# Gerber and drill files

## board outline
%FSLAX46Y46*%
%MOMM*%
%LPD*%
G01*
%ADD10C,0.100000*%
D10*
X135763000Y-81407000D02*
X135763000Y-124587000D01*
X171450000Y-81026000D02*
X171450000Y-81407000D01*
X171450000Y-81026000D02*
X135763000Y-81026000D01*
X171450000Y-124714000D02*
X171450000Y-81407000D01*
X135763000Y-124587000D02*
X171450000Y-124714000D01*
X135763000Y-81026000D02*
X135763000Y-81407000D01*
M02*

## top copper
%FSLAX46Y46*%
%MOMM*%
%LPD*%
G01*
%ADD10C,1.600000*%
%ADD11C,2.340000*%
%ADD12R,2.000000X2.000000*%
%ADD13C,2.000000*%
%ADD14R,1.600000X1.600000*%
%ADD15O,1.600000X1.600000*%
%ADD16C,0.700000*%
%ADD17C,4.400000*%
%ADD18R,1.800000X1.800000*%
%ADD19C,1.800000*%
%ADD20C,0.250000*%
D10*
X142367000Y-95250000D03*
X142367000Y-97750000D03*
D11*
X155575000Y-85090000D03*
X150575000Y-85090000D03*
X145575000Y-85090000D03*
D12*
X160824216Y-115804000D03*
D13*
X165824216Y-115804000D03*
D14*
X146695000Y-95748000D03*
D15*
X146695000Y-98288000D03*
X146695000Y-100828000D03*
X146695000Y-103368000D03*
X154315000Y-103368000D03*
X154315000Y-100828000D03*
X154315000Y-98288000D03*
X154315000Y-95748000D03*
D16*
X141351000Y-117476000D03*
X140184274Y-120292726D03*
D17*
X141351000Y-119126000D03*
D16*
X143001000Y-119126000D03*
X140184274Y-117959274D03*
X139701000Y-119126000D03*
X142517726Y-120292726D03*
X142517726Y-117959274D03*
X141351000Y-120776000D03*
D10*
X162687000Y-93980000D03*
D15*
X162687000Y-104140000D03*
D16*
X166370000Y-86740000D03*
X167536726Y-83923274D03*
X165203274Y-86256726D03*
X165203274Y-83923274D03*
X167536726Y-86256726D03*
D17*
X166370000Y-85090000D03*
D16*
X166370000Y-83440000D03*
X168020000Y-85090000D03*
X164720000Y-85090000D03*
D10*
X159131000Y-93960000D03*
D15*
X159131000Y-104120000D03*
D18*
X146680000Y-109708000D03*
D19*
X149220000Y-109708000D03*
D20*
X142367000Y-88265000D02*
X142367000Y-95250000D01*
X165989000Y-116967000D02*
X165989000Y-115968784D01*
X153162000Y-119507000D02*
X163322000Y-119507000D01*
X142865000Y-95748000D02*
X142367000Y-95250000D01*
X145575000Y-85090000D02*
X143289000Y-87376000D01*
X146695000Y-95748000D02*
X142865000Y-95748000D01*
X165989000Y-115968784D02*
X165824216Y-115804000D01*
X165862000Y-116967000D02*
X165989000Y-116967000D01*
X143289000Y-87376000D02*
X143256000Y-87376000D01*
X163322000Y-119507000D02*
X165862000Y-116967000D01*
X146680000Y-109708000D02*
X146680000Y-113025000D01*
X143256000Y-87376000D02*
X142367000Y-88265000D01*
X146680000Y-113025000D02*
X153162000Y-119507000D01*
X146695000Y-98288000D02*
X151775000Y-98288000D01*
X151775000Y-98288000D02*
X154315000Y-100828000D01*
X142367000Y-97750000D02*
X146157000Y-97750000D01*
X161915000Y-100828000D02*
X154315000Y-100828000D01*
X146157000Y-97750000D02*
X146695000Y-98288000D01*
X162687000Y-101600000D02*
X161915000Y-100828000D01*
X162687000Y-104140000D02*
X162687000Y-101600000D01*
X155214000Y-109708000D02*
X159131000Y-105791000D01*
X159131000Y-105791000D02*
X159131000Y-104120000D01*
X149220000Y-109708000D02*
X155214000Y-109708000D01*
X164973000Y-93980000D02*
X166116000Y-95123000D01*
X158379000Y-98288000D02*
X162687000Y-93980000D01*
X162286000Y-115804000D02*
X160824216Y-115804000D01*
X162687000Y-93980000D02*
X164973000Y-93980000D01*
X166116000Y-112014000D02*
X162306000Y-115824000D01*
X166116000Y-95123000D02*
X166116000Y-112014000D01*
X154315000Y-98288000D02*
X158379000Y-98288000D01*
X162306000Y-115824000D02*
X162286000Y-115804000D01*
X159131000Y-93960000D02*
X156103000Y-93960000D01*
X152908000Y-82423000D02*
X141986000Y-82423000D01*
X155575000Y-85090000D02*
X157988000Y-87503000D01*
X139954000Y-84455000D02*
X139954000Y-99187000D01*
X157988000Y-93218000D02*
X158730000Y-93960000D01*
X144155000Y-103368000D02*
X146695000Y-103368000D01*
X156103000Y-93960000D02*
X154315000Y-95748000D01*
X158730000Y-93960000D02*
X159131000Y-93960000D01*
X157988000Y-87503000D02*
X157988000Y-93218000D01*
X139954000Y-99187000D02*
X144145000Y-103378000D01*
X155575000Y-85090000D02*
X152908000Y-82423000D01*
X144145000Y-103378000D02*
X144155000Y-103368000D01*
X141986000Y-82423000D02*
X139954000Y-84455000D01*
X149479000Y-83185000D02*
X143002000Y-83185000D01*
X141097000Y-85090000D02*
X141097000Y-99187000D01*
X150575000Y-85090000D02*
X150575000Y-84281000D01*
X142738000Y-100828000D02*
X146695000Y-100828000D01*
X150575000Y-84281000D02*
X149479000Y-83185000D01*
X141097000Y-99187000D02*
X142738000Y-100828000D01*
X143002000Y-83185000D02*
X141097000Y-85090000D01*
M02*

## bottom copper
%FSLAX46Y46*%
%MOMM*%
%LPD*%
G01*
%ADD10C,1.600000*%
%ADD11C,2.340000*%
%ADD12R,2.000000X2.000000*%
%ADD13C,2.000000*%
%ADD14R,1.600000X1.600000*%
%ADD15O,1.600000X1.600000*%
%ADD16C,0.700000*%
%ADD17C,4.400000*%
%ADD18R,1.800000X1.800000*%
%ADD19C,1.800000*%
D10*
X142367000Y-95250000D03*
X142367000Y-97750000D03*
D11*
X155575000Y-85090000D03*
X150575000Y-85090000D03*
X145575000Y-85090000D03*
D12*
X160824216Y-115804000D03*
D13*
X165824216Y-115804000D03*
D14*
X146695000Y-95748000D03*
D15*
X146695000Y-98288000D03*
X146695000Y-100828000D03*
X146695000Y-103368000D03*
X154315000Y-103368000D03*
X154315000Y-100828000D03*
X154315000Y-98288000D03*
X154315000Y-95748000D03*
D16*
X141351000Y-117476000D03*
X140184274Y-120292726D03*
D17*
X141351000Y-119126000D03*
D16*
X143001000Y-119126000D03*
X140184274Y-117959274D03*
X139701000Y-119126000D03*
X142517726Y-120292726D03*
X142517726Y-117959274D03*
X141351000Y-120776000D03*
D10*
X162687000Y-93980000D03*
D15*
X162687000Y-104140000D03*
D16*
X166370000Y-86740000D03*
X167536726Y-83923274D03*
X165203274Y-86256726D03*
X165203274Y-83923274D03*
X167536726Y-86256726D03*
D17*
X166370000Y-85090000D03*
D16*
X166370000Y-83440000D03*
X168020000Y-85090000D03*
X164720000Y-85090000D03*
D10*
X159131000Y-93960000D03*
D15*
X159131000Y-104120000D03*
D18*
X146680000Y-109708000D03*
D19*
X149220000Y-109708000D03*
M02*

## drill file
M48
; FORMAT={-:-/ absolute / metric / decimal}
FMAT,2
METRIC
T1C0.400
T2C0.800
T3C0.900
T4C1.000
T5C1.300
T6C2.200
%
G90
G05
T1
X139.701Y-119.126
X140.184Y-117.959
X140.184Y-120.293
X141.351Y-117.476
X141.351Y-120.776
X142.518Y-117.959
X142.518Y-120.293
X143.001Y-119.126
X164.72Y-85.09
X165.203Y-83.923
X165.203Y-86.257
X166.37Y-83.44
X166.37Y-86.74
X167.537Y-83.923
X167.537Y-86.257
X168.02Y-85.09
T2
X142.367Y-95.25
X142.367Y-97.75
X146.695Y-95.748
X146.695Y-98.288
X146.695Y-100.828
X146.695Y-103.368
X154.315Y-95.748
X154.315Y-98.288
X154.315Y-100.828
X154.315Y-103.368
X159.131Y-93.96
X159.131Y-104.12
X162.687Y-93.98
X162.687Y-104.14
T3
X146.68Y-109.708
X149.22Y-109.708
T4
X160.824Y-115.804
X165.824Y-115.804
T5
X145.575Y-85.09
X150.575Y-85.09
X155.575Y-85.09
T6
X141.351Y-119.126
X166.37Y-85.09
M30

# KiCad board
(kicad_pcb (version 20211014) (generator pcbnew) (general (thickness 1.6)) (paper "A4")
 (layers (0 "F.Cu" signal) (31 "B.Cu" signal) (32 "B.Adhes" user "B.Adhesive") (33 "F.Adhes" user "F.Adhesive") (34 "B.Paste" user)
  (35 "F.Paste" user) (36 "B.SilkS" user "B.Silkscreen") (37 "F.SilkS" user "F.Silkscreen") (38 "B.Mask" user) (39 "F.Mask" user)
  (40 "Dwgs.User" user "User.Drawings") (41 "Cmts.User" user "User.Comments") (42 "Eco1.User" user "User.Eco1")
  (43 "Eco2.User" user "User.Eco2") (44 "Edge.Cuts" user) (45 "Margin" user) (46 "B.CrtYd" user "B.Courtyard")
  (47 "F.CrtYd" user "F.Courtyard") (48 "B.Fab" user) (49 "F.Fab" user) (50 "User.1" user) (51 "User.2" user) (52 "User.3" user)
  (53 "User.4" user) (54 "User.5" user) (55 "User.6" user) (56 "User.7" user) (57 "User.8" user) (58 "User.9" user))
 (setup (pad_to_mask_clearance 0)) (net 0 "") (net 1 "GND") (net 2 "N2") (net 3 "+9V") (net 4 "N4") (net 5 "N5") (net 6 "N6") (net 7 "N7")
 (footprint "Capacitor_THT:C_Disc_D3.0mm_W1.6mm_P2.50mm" (layer "F.Cu") (at 142.367 95.25 -90)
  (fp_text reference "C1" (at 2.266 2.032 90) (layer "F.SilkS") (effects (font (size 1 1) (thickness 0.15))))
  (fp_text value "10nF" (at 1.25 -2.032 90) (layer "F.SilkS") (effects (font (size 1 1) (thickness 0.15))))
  (pad "1" thru_hole circle (at 0 0 270) (size 1.6 1.6) (drill 0.8) (layers *.Cu *.Mask) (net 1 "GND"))
  (pad "2" thru_hole circle (at 2.5 0 270) (size 1.6 1.6) (drill 0.8) (layers *.Cu *.Mask) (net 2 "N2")))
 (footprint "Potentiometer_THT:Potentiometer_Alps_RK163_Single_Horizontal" (layer "F.Cu") (at 155.575 85.09 90)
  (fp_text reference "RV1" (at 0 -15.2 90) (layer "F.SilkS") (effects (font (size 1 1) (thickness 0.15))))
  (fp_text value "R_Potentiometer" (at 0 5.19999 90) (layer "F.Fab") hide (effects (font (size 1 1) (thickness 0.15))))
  (pad "1" thru_hole circle (at 0 0 90) (size 2.34 2.34) (drill 1.3) (layers *.Cu *.Mask) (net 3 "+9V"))
  (pad "2" thru_hole circle (at 0 -5 90) (size 2.34 2.34) (drill 1.3) (layers *.Cu *.Mask) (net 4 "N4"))
  (pad "3" thru_hole circle (at 0 -10 90) (size 2.34 2.34) (drill 1.3) (layers *.Cu *.Mask) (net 1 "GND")))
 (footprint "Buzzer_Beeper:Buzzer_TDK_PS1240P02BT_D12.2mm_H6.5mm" (layer "F.Cu") (at 160.824216 115.804)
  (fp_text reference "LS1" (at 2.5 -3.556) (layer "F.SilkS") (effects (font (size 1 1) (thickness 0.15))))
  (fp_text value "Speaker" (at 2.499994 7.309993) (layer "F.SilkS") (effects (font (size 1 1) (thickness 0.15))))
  (pad "1" thru_hole rect (at 0 0) (size 2 2) (drill 1) (layers *.Cu *.Mask) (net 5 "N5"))
  (pad "2" thru_hole circle (at 5 0) (size 2 2) (drill 1) (layers *.Cu *.Mask) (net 1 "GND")))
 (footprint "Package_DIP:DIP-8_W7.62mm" (layer "F.Cu") (at 146.695 95.748)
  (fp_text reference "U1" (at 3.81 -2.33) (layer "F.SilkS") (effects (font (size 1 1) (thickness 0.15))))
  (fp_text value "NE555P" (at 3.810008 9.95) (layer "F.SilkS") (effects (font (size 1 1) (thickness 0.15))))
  (pad "1" thru_hole rect (at 0 0) (size 1.6 1.6) (drill 0.8) (layers *.Cu *.Mask) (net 1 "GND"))
  (pad "2" thru_hole oval (at 0 2.54) (size 1.6 1.6) (drill 0.8) (layers *.Cu *.Mask) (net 2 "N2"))
  (pad "3" thru_hole oval (at 0 5.08) (size 1.6 1.6) (drill 0.8) (layers *.Cu *.Mask) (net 4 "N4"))
  (pad "4" thru_hole oval (at 0 7.62) (size 1.6 1.6) (drill 0.8) (layers *.Cu *.Mask) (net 3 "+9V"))
  (pad "5" thru_hole oval (at 7.62 7.62) (size 1.6 1.6) (drill 0.8) (layers *.Cu *.Mask) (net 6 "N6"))
  (pad "6" thru_hole oval (at 7.62 5.08) (size 1.6 1.6) (drill 0.8) (layers *.Cu *.Mask) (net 2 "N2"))
  (pad "7" thru_hole oval (at 7.62 2.54) (size 1.6 1.6) (drill 0.8) (layers *.Cu *.Mask) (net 5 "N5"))
  (pad "8" thru_hole oval (at 7.62 0) (size 1.6 1.6) (drill 0.8) (layers *.Cu *.Mask) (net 3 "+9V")))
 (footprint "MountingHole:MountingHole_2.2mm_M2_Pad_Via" (layer "F.Cu") (at 141.351 119.126)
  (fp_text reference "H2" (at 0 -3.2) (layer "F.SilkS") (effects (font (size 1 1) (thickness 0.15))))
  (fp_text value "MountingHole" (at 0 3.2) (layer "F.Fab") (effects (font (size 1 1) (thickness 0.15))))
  (pad "1" thru_hole circle (at 0 -1.65) (size 0.7 0.7) (drill 0.4) (layers *.Cu *.Mask))
  (pad "1" thru_hole circle (at -1.166726 1.166726) (size 0.7 0.7) (drill 0.4) (layers *.Cu *.Mask))
  (pad "1" thru_hole circle (at 0 0) (size 4.4 4.4) (drill 2.2) (layers *.Cu *.Mask))
  (pad "1" thru_hole circle (at 1.65 0) (size 0.7 0.7) (drill 0.4) (layers *.Cu *.Mask))
  (pad "1" thru_hole circle (at -1.166726 -1.166726) (size 0.7 0.7) (drill 0.4) (layers *.Cu *.Mask))
  (pad "1" thru_hole circle (at -1.65 0) (size 0.7 0.7) (drill 0.4) (layers *.Cu *.Mask))
  (pad "1" thru_hole circle (at 1.166726 1.166726) (size 0.7 0.7) (drill 0.4) (layers *.Cu *.Mask))
  (pad "1" thru_hole circle (at 1.166726 -1.166726) (size 0.7 0.7) (drill 0.4) (layers *.Cu *.Mask))
  (pad "1" thru_hole circle (at 0 1.65) (size 0.7 0.7) (drill 0.4) (layers *.Cu *.Mask)))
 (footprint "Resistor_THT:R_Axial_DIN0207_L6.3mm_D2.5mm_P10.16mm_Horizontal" (layer "F.Cu") (at 162.687 93.98 -90)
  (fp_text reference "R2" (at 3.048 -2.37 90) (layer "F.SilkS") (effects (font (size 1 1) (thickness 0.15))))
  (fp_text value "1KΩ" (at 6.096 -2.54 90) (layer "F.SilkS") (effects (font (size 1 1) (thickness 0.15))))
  (pad "1" thru_hole circle (at 0 0 270) (size 1.6 1.6) (drill 0.8) (layers *.Cu *.Mask) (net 5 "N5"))
  (pad "2" thru_hole oval (at 10.16 0 270) (size 1.6 1.6) (drill 0.8) (layers *.Cu *.Mask) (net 2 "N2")))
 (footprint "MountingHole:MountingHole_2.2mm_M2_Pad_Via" (layer "F.Cu") (at 166.37 85.09)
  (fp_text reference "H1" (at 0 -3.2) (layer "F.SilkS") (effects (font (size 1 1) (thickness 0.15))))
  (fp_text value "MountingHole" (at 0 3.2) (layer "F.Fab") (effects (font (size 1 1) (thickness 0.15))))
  (pad "1" thru_hole circle (at 0 1.65) (size 0.7 0.7) (drill 0.4) (layers *.Cu *.Mask))
  (pad "1" thru_hole circle (at 1.166726 -1.166726) (size 0.7 0.7) (drill 0.4) (layers *.Cu *.Mask))
  (pad "1" thru_hole circle (at -1.166726 1.166726) (size 0.7 0.7) (drill 0.4) (layers *.Cu *.Mask))
  (pad "1" thru_hole circle (at -1.166726 -1.166726) (size 0.7 0.7) (drill 0.4) (layers *.Cu *.Mask))
  (pad "1" thru_hole circle (at 1.166726 1.166726) (size 0.7 0.7) (drill 0.4) (layers *.Cu *.Mask))
  (pad "1" thru_hole circle (at 0 0) (size 4.4 4.4) (drill 2.2) (layers *.Cu *.Mask))
  (pad "1" thru_hole circle (at 0 -1.65) (size 0.7 0.7) (drill 0.4) (layers *.Cu *.Mask))
  (pad "1" thru_hole circle (at 1.65 0) (size 0.7 0.7) (drill 0.4) (layers *.Cu *.Mask))
  (pad "1" thru_hole circle (at -1.65 0) (size 0.7 0.7) (drill 0.4) (layers *.Cu *.Mask)))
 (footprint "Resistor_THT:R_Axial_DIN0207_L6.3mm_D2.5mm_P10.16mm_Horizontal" (layer "F.Cu") (at 159.131 93.96 -90)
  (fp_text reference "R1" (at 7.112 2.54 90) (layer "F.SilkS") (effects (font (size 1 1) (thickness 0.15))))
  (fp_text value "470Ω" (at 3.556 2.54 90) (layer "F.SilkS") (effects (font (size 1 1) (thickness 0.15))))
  (pad "1" thru_hole circle (at 0 0 270) (size 1.6 1.6) (drill 0.8) (layers *.Cu *.Mask) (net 3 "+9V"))
  (pad "2" thru_hole oval (at 10.16 0 270) (size 1.6 1.6) (drill 0.8) (layers *.Cu *.Mask) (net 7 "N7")))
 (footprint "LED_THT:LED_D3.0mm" (layer "F.Cu") (at 146.68 109.708)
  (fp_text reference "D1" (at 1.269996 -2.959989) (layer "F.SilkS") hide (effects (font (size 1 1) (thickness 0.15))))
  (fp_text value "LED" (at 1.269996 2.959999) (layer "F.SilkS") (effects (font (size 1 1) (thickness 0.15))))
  (pad "1" thru_hole rect (at 0 0) (size 1.8 1.8) (drill 0.9) (layers *.Cu *.Mask) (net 1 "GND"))
  (pad "2" thru_hole circle (at 2.54 0) (size 1.8 1.8) (drill 0.9) (layers *.Cu *.Mask) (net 7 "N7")))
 (gr_line (start 135.763 81.407) (end 135.763 124.587) (layer "Edge.Cuts") (width 0.1))
 (gr_line (start 171.45 81.026) (end 171.45 81.407) (layer "Edge.Cuts") (width 0.1))
 (gr_line (start 171.45 81.026) (end 135.763 81.026) (layer "Edge.Cuts") (width 0.1))
 (gr_line (start 171.45 124.714) (end 171.45 81.407) (layer "Edge.Cuts") (width 0.1))
 (gr_line (start 135.763 124.587) (end 171.45 124.714) (layer "Edge.Cuts") (width 0.1))
 (gr_line (start 135.763 81.026) (end 135.763 81.407) (layer "Edge.Cuts") (width 0.1))
 (segment (start 142.367 88.265) (end 142.367 95.25) (width 0.25) (layer "F.Cu") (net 1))
 (segment (start 165.989 116.967) (end 165.989 115.968784) (width 0.25) (layer "F.Cu") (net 1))
 (segment (start 153.162 119.507) (end 163.322 119.507) (width 0.25) (layer "F.Cu") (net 1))
 (segment (start 142.865 95.748) (end 142.367 95.25) (width 0.25) (layer "F.Cu") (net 1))
 (segment (start 145.575 85.09) (end 143.289 87.376) (width 0.25) (layer "F.Cu") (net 1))
 (segment (start 146.695 95.748) (end 142.865 95.748) (width 0.25) (layer "F.Cu") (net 1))
 (segment (start 165.989 115.968784) (end 165.824216 115.804) (width 0.25) (layer "F.Cu") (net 1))
 (segment (start 165.862 116.967) (end 165.989 116.967) (width 0.25) (layer "F.Cu") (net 1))
 (segment (start 143.289 87.376) (end 143.256 87.376) (width 0.25) (layer "F.Cu") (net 1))
 (segment (start 163.322 119.507) (end 165.862 116.967) (width 0.25) (layer "F.Cu") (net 1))
 (segment (start 146.68 109.708) (end 146.68 113.025) (width 0.25) (layer "F.Cu") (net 1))
 (segment (start 143.256 87.376) (end 142.367 88.265) (width 0.25) (layer "F.Cu") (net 1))
 (segment (start 146.68 113.025) (end 153.162 119.507) (width 0.25) (layer "F.Cu") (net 1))
 (segment (start 146.695 98.288) (end 151.775 98.288) (width 0.25) (layer "F.Cu") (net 2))
 (segment (start 151.775 98.288) (end 154.315 100.828) (width 0.25) (layer "F.Cu") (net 2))
 (segment (start 142.367 97.75) (end 146.157 97.75) (width 0.25) (layer "F.Cu") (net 2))
 (segment (start 161.915 100.828) (end 154.315 100.828) (width 0.25) (layer "F.Cu") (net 2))
 (segment (start 146.157 97.75) (end 146.695 98.288) (width 0.25) (layer "F.Cu") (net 2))
 (segment (start 162.687 101.6) (end 161.915 100.828) (width 0.25) (layer "F.Cu") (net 2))
 (segment (start 162.687 104.14) (end 162.687 101.6) (width 0.25) (layer "F.Cu") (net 2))
 (segment (start 155.214 109.708) (end 159.131 105.791) (width 0.25) (layer "F.Cu") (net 7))
 (segment (start 159.131 105.791) (end 159.131 104.12) (width 0.25) (layer "F.Cu") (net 7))
 (segment (start 149.22 109.708) (end 155.214 109.708) (width 0.25) (layer "F.Cu") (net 7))
 (segment (start 164.973 93.98) (end 166.116 95.123) (width 0.25) (layer "F.Cu") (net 5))
 (segment (start 158.379 98.288) (end 162.687 93.98) (width 0.25) (layer "F.Cu") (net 5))
 (segment (start 162.286 115.804) (end 160.824216 115.804) (width 0.25) (layer "F.Cu") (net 5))
 (segment (start 162.687 93.98) (end 164.973 93.98) (width 0.25) (layer "F.Cu") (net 5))
 (segment (start 166.116 112.014) (end 162.306 115.824) (width 0.25) (layer "F.Cu") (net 5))
 (segment (start 166.116 95.123) (end 166.116 112.014) (width 0.25) (layer "F.Cu") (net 5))
 (segment (start 154.315 98.288) (end 158.379 98.288) (width 0.25) (layer "F.Cu") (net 5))
 (segment (start 162.306 115.824) (end 162.286 115.804) (width 0.25) (layer "F.Cu") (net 5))
 (segment (start 159.131 93.96) (end 156.103 93.96) (width 0.25) (layer "F.Cu") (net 3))
 (segment (start 152.908 82.423) (end 141.986 82.423) (width 0.25) (layer "F.Cu") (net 3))
 (segment (start 155.575 85.09) (end 157.988 87.503) (width 0.25) (layer "F.Cu") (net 3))
 (segment (start 139.954 84.455) (end 139.954 99.187) (width 0.25) (layer "F.Cu") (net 3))
 (segment (start 157.988 93.218) (end 158.73 93.96) (width 0.25) (layer "F.Cu") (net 3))
 (segment (start 144.155 103.368) (end 146.695 103.368) (width 0.25) (layer "F.Cu") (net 3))
 (segment (start 156.103 93.96) (end 154.315 95.748) (width 0.25) (layer "F.Cu") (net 3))
 (segment (start 158.73 93.96) (end 159.131 93.96) (width 0.25) (layer "F.Cu") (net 3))
 (segment (start 157.988 87.503) (end 157.988 93.218) (width 0.25) (layer "F.Cu") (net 3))
 (segment (start 139.954 99.187) (end 144.145 103.378) (width 0.25) (layer "F.Cu") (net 3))
 (segment (start 155.575 85.09) (end 152.908 82.423) (width 0.25) (layer "F.Cu") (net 3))
 (segment (start 144.145 103.378) (end 144.155 103.368) (width 0.25) (layer "F.Cu") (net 3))
 (segment (start 141.986 82.423) (end 139.954 84.455) (width 0.25) (layer "F.Cu") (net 3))
 (segment (start 149.479 83.185) (end 143.002 83.185) (width 0.25) (layer "F.Cu") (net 4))
 (segment (start 141.097 85.09) (end 141.097 99.187) (width 0.25) (layer "F.Cu") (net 4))
 (segment (start 150.575 85.09) (end 150.575 84.281) (width 0.25) (layer "F.Cu") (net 4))
 (segment (start 142.738 100.828) (end 146.695 100.828) (width 0.25) (layer "F.Cu") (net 4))
 (segment (start 150.575 84.281) (end 149.479 83.185) (width 0.25) (layer "F.Cu") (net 4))
 (segment (start 141.097 99.187) (end 142.738 100.828) (width 0.25) (layer "F.Cu") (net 4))
 (segment (start 143.002 83.185) (end 141.097 85.09) (width 0.25) (layer "F.Cu") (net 4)))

